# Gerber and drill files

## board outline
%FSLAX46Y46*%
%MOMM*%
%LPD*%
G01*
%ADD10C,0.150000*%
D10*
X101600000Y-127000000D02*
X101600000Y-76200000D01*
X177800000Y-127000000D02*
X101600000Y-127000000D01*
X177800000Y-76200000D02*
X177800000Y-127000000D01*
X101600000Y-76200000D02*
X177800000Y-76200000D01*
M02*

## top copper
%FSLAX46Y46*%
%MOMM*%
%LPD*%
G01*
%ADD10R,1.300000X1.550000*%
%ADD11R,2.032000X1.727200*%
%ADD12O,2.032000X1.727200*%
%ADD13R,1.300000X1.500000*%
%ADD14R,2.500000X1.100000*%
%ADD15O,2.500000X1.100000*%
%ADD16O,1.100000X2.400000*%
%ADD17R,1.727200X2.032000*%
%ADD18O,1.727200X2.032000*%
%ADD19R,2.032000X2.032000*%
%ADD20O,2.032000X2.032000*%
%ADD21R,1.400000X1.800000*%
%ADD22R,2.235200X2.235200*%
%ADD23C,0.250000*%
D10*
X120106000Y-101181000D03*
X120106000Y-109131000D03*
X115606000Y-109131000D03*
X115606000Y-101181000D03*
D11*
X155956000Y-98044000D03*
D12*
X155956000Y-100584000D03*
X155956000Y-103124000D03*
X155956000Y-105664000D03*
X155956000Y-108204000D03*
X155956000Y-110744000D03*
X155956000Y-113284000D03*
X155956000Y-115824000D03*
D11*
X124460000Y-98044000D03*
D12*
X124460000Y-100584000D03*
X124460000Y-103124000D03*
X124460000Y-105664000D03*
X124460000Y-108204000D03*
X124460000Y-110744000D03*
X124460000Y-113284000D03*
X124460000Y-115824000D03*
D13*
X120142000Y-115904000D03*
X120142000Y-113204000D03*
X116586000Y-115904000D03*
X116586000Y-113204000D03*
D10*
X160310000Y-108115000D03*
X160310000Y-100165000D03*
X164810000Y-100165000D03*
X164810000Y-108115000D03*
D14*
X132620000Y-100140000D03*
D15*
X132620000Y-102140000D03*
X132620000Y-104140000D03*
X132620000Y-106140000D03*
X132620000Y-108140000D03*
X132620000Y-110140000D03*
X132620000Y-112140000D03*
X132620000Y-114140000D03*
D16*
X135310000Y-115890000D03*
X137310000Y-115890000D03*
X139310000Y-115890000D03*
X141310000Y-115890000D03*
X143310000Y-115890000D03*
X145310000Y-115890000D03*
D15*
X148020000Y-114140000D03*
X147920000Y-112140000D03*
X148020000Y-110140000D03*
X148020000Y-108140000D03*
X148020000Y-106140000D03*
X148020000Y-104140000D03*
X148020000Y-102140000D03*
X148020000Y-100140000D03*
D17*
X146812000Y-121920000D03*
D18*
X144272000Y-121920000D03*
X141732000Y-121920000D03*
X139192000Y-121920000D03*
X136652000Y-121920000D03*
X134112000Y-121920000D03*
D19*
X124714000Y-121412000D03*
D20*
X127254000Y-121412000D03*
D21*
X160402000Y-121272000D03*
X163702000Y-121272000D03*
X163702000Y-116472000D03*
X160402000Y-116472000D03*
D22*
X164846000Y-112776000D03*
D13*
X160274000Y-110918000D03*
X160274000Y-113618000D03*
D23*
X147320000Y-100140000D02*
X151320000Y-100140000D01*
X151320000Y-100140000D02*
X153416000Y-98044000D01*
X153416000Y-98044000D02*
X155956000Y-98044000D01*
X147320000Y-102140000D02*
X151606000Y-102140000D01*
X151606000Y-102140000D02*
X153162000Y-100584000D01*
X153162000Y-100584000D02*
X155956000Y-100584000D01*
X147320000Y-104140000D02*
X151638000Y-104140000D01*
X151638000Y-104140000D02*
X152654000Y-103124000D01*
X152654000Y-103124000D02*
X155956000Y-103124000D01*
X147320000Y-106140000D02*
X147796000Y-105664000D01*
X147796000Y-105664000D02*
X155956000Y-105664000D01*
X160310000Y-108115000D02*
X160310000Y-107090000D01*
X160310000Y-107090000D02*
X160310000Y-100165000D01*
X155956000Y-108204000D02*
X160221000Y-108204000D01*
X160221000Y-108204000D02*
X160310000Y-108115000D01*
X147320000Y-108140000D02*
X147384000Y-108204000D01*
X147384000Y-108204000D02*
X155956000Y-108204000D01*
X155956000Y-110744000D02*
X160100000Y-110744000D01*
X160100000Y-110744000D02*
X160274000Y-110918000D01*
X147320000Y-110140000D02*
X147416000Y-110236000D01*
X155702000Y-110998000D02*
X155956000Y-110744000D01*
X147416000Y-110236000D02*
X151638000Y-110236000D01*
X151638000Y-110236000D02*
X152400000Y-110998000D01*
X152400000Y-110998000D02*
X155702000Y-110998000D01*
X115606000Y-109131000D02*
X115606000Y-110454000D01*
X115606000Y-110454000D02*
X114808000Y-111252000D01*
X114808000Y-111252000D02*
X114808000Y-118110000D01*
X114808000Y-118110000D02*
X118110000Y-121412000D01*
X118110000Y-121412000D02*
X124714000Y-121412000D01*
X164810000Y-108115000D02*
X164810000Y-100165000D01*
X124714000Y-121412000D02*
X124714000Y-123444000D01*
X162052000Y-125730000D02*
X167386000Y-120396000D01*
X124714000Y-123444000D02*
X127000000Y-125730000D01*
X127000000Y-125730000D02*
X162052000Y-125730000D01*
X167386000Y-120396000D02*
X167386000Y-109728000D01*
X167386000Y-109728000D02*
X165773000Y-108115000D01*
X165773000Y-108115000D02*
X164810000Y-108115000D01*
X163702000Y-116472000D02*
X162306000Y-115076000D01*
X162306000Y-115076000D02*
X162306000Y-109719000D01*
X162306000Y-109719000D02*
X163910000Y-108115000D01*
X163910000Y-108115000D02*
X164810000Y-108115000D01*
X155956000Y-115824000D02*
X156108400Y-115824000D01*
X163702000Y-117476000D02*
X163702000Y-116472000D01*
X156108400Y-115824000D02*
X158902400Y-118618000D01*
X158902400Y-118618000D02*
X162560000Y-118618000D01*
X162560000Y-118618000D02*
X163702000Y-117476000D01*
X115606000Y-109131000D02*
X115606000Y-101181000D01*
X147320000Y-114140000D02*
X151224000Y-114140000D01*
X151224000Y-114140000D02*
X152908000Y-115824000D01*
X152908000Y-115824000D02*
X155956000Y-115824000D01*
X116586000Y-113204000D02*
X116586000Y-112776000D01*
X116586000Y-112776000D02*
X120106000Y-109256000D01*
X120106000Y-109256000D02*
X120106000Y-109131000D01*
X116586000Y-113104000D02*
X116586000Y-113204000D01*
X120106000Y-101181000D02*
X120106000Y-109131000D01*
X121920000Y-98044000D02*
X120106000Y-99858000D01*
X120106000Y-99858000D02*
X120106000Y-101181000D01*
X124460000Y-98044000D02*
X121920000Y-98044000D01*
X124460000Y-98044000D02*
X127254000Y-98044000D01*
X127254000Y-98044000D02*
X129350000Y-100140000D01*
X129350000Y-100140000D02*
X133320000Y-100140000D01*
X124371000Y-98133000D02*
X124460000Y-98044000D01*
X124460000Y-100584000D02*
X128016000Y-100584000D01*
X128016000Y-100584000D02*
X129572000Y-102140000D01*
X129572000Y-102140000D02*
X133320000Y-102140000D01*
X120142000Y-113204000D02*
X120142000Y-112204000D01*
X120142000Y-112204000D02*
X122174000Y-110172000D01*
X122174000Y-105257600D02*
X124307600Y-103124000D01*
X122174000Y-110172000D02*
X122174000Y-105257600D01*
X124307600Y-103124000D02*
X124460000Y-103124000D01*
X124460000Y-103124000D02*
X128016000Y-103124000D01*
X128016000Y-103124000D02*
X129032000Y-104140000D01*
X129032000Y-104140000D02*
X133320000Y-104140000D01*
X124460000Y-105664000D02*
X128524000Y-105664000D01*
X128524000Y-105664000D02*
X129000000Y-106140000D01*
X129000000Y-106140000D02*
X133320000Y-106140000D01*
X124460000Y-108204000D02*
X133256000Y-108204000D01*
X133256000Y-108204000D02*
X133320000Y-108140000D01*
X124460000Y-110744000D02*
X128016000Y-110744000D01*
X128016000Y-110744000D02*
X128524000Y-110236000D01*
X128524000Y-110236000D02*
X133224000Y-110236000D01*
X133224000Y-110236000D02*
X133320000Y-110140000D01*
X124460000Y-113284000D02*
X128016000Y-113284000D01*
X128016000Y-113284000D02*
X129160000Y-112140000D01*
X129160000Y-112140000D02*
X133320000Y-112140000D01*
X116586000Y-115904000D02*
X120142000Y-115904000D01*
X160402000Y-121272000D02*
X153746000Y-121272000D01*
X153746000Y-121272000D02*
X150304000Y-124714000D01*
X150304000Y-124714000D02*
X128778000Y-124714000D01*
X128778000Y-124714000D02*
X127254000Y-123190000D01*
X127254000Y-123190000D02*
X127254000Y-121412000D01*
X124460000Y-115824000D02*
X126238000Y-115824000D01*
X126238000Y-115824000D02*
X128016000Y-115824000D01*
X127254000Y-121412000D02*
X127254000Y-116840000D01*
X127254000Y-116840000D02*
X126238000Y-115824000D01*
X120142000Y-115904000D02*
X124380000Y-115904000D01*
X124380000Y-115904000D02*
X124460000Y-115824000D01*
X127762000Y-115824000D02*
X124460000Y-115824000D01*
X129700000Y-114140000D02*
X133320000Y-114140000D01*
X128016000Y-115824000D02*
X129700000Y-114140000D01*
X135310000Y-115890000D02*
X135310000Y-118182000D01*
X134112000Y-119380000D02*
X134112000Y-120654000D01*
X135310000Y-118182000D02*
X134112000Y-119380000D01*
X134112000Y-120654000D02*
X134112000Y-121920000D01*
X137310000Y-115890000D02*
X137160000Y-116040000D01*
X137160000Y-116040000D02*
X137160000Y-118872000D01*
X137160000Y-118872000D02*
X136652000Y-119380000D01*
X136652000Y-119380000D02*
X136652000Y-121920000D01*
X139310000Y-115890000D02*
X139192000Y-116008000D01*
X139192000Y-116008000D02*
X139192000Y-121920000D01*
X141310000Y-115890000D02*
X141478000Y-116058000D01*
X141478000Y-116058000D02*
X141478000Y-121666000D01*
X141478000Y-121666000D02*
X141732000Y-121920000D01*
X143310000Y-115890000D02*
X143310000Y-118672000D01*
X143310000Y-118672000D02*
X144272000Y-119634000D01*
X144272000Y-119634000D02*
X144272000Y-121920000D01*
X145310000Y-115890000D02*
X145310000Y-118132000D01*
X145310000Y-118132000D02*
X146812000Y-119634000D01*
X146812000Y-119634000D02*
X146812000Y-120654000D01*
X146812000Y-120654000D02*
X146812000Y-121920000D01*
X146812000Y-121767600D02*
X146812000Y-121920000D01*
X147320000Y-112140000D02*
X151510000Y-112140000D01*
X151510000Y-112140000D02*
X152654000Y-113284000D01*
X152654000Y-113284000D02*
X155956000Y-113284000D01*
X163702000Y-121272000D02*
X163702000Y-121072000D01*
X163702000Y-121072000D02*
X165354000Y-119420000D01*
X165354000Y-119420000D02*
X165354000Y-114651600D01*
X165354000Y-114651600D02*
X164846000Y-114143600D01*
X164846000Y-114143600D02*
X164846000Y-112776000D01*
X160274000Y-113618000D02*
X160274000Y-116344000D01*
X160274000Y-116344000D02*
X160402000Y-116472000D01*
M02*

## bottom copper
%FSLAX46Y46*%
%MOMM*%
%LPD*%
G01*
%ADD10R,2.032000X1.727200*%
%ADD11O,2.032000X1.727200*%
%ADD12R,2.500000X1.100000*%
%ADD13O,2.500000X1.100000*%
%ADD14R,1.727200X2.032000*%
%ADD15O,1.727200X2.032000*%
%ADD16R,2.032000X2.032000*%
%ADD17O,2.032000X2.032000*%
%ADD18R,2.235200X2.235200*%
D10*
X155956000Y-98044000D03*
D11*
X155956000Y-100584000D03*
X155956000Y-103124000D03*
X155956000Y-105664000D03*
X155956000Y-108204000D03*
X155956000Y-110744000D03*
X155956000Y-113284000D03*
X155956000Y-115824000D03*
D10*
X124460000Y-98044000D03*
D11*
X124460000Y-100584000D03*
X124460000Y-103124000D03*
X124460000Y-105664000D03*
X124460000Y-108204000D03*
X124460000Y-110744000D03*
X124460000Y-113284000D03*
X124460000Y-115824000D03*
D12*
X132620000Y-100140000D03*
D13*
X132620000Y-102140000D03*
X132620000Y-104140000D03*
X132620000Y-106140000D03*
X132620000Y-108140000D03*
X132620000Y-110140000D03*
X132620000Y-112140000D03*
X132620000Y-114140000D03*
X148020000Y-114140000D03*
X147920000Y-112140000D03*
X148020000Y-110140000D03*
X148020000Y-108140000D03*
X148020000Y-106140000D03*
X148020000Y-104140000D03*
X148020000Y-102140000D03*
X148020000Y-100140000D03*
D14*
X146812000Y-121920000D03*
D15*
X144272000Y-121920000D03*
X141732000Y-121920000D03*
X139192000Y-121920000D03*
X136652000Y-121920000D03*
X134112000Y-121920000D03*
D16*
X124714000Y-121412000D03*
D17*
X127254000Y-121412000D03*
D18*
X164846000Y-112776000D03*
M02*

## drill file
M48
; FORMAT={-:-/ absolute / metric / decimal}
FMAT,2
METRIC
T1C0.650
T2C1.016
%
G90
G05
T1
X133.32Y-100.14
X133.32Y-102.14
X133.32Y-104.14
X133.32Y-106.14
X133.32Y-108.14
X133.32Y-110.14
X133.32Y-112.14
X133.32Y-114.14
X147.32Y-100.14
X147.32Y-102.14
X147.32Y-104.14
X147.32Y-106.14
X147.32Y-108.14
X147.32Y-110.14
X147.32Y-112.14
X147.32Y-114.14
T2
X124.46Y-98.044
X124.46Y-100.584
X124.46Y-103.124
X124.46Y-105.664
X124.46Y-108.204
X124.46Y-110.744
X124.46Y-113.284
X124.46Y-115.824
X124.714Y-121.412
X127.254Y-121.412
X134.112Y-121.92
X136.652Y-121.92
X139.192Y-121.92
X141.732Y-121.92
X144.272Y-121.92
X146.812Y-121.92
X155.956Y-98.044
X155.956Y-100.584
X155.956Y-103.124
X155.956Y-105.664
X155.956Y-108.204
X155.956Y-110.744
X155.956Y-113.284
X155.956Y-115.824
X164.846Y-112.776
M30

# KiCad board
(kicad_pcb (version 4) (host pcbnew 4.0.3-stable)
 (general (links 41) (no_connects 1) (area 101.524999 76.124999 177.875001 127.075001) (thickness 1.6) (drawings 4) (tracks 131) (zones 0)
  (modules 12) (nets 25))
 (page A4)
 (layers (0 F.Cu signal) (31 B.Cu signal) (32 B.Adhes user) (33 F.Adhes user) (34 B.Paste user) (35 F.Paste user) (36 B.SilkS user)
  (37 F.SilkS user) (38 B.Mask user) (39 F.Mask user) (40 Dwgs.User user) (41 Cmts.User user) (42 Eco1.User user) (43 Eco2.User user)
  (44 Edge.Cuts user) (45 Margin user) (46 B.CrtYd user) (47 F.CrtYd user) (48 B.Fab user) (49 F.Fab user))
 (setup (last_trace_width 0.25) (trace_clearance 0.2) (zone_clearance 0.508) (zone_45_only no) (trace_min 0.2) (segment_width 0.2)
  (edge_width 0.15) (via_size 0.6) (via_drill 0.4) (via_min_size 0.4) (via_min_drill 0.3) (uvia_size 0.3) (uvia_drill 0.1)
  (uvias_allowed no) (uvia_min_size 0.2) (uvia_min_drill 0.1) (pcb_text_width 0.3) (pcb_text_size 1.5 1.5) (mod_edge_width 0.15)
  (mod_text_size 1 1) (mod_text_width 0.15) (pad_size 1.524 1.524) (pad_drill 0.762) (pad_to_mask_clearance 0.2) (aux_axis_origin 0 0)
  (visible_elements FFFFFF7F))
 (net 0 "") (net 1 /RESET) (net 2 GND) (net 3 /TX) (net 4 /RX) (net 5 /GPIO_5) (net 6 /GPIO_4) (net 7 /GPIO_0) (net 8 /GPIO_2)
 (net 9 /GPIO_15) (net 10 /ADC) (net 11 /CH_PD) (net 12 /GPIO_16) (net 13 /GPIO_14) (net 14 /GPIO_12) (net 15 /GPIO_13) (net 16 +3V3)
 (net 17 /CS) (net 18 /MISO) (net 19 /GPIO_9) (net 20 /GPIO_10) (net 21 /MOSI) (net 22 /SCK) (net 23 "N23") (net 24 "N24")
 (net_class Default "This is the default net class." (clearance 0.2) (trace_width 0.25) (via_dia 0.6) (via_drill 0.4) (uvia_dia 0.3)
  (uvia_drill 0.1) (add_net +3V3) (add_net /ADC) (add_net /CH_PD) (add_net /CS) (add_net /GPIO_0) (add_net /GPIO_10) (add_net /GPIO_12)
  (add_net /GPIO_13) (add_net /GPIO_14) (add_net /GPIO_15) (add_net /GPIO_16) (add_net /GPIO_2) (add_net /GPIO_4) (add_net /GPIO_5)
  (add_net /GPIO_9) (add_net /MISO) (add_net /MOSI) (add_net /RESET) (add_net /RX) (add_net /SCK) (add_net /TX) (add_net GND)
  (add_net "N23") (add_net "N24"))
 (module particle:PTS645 (layer F.Cu) (at 117.856 105.156 270)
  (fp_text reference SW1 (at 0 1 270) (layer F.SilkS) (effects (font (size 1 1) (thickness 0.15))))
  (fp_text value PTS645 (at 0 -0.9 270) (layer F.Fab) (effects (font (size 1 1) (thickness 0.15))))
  (pad 1 smd rect (at -3.975 -2.25 270) (size 1.55 1.3) (layers F.Cu F.Paste F.Mask) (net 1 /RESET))
  (pad 1 smd rect (at 3.975 -2.25 270) (size 1.55 1.3) (layers F.Cu F.Paste F.Mask) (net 1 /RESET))
  (pad 4 smd rect (at 3.975 2.25 270) (size 1.55 1.3) (layers F.Cu F.Paste F.Mask) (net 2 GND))
  (pad 4 smd rect (at -3.975 2.25 270) (size 1.55 1.3) (layers F.Cu F.Paste F.Mask) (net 2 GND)))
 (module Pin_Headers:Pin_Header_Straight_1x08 (layer F.Cu) (at 155.956 98.044)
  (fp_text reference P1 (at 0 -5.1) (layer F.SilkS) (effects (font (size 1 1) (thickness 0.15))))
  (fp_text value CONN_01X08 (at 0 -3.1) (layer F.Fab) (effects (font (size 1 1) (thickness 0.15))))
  (pad 1 thru_hole rect (at 0 0) (size 2.032 1.7272) (drill 1.016) (layers *.Cu *.Mask F.SilkS) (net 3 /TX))
  (pad 2 thru_hole oval (at 0 2.54) (size 2.032 1.7272) (drill 1.016) (layers *.Cu *.Mask F.SilkS) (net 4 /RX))
  (pad 3 thru_hole oval (at 0 5.08) (size 2.032 1.7272) (drill 1.016) (layers *.Cu *.Mask F.SilkS) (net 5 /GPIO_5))
  (pad 4 thru_hole oval (at 0 7.62) (size 2.032 1.7272) (drill 1.016) (layers *.Cu *.Mask F.SilkS) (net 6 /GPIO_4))
  (pad 5 thru_hole oval (at 0 10.16) (size 2.032 1.7272) (drill 1.016) (layers *.Cu *.Mask F.SilkS) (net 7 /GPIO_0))
  (pad 6 thru_hole oval (at 0 12.7) (size 2.032 1.7272) (drill 1.016) (layers *.Cu *.Mask F.SilkS) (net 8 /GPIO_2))
  (pad 7 thru_hole oval (at 0 15.24) (size 2.032 1.7272) (drill 1.016) (layers *.Cu *.Mask F.SilkS) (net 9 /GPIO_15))
  (pad 8 thru_hole oval (at 0 17.78) (size 2.032 1.7272) (drill 1.016) (layers *.Cu *.Mask F.SilkS) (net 2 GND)))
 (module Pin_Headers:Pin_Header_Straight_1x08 (layer F.Cu) (at 124.46 98.044)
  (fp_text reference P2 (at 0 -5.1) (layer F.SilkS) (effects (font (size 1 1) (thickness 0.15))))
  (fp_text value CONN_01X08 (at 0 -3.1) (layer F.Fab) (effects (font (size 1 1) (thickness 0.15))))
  (pad 1 thru_hole rect (at 0 0) (size 2.032 1.7272) (drill 1.016) (layers *.Cu *.Mask F.SilkS) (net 1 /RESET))
  (pad 2 thru_hole oval (at 0 2.54) (size 2.032 1.7272) (drill 1.016) (layers *.Cu *.Mask F.SilkS) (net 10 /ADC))
  (pad 3 thru_hole oval (at 0 5.08) (size 2.032 1.7272) (drill 1.016) (layers *.Cu *.Mask F.SilkS) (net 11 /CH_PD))
  (pad 4 thru_hole oval (at 0 7.62) (size 2.032 1.7272) (drill 1.016) (layers *.Cu *.Mask F.SilkS) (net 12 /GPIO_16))
  (pad 5 thru_hole oval (at 0 10.16) (size 2.032 1.7272) (drill 1.016) (layers *.Cu *.Mask F.SilkS) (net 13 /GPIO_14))
  (pad 6 thru_hole oval (at 0 12.7) (size 2.032 1.7272) (drill 1.016) (layers *.Cu *.Mask F.SilkS) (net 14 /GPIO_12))
  (pad 7 thru_hole oval (at 0 15.24) (size 2.032 1.7272) (drill 1.016) (layers *.Cu *.Mask F.SilkS) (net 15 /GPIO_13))
  (pad 8 thru_hole oval (at 0 17.78) (size 2.032 1.7272) (drill 1.016) (layers *.Cu *.Mask F.SilkS) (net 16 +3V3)))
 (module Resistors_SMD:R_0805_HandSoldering (layer F.Cu) (at 120.142 114.554 90)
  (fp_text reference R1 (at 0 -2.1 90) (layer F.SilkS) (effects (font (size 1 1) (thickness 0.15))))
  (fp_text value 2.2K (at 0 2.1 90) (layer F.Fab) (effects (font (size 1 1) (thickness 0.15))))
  (pad 1 smd rect (at -1.35 0 90) (size 1.5 1.3) (layers F.Cu F.Paste F.Mask) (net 16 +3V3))
  (pad 2 smd rect (at 1.35 0 90) (size 1.5 1.3) (layers F.Cu F.Paste F.Mask) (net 11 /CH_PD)))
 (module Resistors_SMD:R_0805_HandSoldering (layer F.Cu) (at 116.586 114.554 90)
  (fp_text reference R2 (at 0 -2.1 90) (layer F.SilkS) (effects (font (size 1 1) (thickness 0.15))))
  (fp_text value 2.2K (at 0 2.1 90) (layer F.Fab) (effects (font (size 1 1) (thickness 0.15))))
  (pad 1 smd rect (at -1.35 0 90) (size 1.5 1.3) (layers F.Cu F.Paste F.Mask) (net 16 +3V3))
  (pad 2 smd rect (at 1.35 0 90) (size 1.5 1.3) (layers F.Cu F.Paste F.Mask) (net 1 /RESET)))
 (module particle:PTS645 (layer F.Cu) (at 162.56 104.14 90)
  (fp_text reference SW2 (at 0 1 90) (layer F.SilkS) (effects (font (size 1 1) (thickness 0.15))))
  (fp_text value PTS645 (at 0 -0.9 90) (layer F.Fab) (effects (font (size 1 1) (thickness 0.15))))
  (pad 1 smd rect (at -3.975 -2.25 90) (size 1.55 1.3) (layers F.Cu F.Paste F.Mask) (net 7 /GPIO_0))
  (pad 1 smd rect (at 3.975 -2.25 90) (size 1.55 1.3) (layers F.Cu F.Paste F.Mask) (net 7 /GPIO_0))
  (pad 4 smd rect (at 3.975 2.25 90) (size 1.55 1.3) (layers F.Cu F.Paste F.Mask) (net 2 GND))
  (pad 4 smd rect (at -3.975 2.25 90) (size 1.55 1.3) (layers F.Cu F.Paste F.Mask) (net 2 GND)))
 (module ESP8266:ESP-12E (layer F.Cu) (at 133.32 100.14)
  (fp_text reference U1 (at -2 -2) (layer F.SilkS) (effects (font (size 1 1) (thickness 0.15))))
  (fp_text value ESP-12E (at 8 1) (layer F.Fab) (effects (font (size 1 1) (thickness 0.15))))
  (pad 1 thru_hole rect (at 0 0) (size 2.5 1.1) (drill 0.65 (offset -0.7 0)) (layers *.Cu *.Mask F.SilkS) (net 1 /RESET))
  (pad 2 thru_hole oval (at 0 2) (size 2.5 1.1) (drill 0.65 (offset -0.7 0)) (layers *.Cu *.Mask F.SilkS) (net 10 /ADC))
  (pad 3 thru_hole oval (at 0 4) (size 2.5 1.1) (drill 0.65 (offset -0.7 0)) (layers *.Cu *.Mask F.SilkS) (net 11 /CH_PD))
  (pad 4 thru_hole oval (at 0 6) (size 2.5 1.1) (drill 0.65 (offset -0.7 0)) (layers *.Cu *.Mask F.SilkS) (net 12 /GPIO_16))
  (pad 5 thru_hole oval (at 0 8) (size 2.5 1.1) (drill 0.65 (offset -0.7 0)) (layers *.Cu *.Mask F.SilkS) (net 13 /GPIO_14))
  (pad 6 thru_hole oval (at 0 10) (size 2.5 1.1) (drill 0.65 (offset -0.7 0)) (layers *.Cu *.Mask F.SilkS) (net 14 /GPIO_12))
  (pad 7 thru_hole oval (at 0 12) (size 2.5 1.1) (drill 0.65 (offset -0.7 0)) (layers *.Cu *.Mask F.SilkS) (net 15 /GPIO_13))
  (pad 8 thru_hole oval (at 0 14) (size 2.5 1.1) (drill 0.65 (offset -0.7 0)) (layers *.Cu *.Mask F.SilkS) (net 16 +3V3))
  (pad 9 smd oval (at 1.99 15.75 90) (size 2.4 1.1) (layers F.Cu F.Paste F.Mask) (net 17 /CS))
  (pad 10 smd oval (at 3.99 15.75 90) (size 2.4 1.1) (layers F.Cu F.Paste F.Mask) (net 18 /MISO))
  (pad 11 smd oval (at 5.99 15.75 90) (size 2.4 1.1) (layers F.Cu F.Paste F.Mask) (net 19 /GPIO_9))
  (pad 12 smd oval (at 7.99 15.75 90) (size 2.4 1.1) (layers F.Cu F.Paste F.Mask) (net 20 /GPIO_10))
  (pad 13 smd oval (at 9.99 15.75 90) (size 2.4 1.1) (layers F.Cu F.Paste F.Mask) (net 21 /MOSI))
  (pad 14 smd oval (at 11.99 15.75 90) (size 2.4 1.1) (layers F.Cu F.Paste F.Mask) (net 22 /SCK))
  (pad 15 thru_hole oval (at 14 14) (size 2.5 1.1) (drill 0.65 (offset 0.7 0)) (layers *.Cu *.Mask F.SilkS) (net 2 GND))
  (pad 16 thru_hole oval (at 14 12) (size 2.5 1.1) (drill 0.65 (offset 0.6 0)) (layers *.Cu *.Mask F.SilkS) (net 9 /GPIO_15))
  (pad 17 thru_hole oval (at 14 10) (size 2.5 1.1) (drill 0.65 (offset 0.7 0)) (layers *.Cu *.Mask F.SilkS) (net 8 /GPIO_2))
  (pad 18 thru_hole oval (at 14 8) (size 2.5 1.1) (drill 0.65 (offset 0.7 0)) (layers *.Cu *.Mask F.SilkS) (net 7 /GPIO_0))
  (pad 19 thru_hole oval (at 14 6) (size 2.5 1.1) (drill 0.65 (offset 0.7 0)) (layers *.Cu *.Mask F.SilkS) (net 6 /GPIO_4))
  (pad 20 thru_hole oval (at 14 4) (size 2.5 1.1) (drill 0.65 (offset 0.7 0)) (layers *.Cu *.Mask F.SilkS) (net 5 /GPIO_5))
  (pad 21 thru_hole oval (at 14 2) (size 2.5 1.1) (drill 0.65 (offset 0.7 0)) (layers *.Cu *.Mask F.SilkS) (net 4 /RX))
  (pad 22 thru_hole oval (at 14 0) (size 2.5 1.1) (drill 0.65 (offset 0.7 0)) (layers *.Cu *.Mask F.SilkS) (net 3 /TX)))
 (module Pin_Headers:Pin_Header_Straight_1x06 (layer F.Cu) (at 146.812 121.92 270)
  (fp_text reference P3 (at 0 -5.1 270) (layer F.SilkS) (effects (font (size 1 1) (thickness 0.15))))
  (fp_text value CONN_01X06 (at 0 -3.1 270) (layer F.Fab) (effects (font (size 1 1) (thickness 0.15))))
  (pad 1 thru_hole rect (at 0 0 270) (size 2.032 1.7272) (drill 1.016) (layers *.Cu *.Mask F.SilkS) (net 22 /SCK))
  (pad 2 thru_hole oval (at 0 2.54 270) (size 2.032 1.7272) (drill 1.016) (layers *.Cu *.Mask F.SilkS) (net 21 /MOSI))
  (pad 3 thru_hole oval (at 0 5.08 270) (size 2.032 1.7272) (drill 1.016) (layers *.Cu *.Mask F.SilkS) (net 20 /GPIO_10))
  (pad 4 thru_hole oval (at 0 7.62 270) (size 2.032 1.7272) (drill 1.016) (layers *.Cu *.Mask F.SilkS) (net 19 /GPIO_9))
  (pad 5 thru_hole oval (at 0 10.16 270) (size 2.032 1.7272) (drill 1.016) (layers *.Cu *.Mask F.SilkS) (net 18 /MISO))
  (pad 6 thru_hole oval (at 0 12.7 270) (size 2.032 1.7272) (drill 1.016) (layers *.Cu *.Mask F.SilkS) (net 17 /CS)))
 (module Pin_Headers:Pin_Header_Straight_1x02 (layer F.Cu) (at 124.714 121.412 90)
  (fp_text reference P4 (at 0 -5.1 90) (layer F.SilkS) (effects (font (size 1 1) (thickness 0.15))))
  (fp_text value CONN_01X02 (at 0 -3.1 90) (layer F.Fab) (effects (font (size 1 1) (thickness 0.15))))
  (pad 1 thru_hole rect (at 0 0 90) (size 2.032 2.032) (drill 1.016) (layers *.Cu *.Mask F.SilkS) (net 2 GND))
  (pad 2 thru_hole oval (at 0 2.54 90) (size 2.032 2.032) (drill 1.016) (layers *.Cu *.Mask F.SilkS) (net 16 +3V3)))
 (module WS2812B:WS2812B (layer F.Cu) (at 162.052 118.872 180)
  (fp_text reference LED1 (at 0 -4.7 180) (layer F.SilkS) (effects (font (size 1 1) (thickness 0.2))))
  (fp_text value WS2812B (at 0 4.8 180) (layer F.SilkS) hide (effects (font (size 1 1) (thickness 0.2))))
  (pad 1 smd rect (at 1.65 -2.4 180) (size 1.4 1.8) (layers F.Cu F.Paste F.Mask) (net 16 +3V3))
  (pad 2 smd rect (at -1.65 -2.4 180) (size 1.4 1.8) (layers F.Cu F.Paste F.Mask) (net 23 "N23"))
  (pad 3 smd rect (at -1.65 2.4 180) (size 1.4 1.8) (layers F.Cu F.Paste F.Mask) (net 2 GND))
  (pad 4 smd rect (at 1.65 2.4 180) (size 1.4 1.8) (layers F.Cu F.Paste F.Mask) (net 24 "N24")))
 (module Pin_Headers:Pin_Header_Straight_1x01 (layer F.Cu) (at 164.846 112.776)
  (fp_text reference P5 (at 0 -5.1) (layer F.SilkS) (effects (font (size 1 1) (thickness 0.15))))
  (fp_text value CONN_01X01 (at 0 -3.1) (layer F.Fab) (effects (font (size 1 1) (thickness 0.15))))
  (pad 1 thru_hole rect (at 0 0) (size 2.2352 2.2352) (drill 1.016) (layers *.Cu *.Mask F.SilkS) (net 23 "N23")))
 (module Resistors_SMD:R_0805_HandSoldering (layer F.Cu) (at 160.274 112.268 270)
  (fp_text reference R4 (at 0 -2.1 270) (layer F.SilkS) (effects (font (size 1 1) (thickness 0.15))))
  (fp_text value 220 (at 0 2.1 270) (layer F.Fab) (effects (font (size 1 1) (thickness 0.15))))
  (pad 1 smd rect (at -1.35 0 270) (size 1.5 1.3) (layers F.Cu F.Paste F.Mask) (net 8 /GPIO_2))
  (pad 2 smd rect (at 1.35 0 270) (size 1.5 1.3) (layers F.Cu F.Paste F.Mask) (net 24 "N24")))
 (gr_line (start 101.6 127) (end 101.6 76.2) (layer Edge.Cuts) (width 0.15))
 (gr_line (start 177.8 127) (end 101.6 127) (layer Edge.Cuts) (width 0.15))
 (gr_line (start 177.8 76.2) (end 177.8 127) (layer Edge.Cuts) (width 0.15))
 (gr_line (start 101.6 76.2) (end 177.8 76.2) (layer Edge.Cuts) (width 0.15))
 (segment (start 147.32 100.14) (end 151.32 100.14) (width 0.25) (layer F.Cu) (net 3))
 (segment (start 151.32 100.14) (end 153.416 98.044) (width 0.25) (layer F.Cu) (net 3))
 (segment (start 153.416 98.044) (end 155.956 98.044) (width 0.25) (layer F.Cu) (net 3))
 (segment (start 147.32 102.14) (end 151.606 102.14) (width 0.25) (layer F.Cu) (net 4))
 (segment (start 151.606 102.14) (end 153.162 100.584) (width 0.25) (layer F.Cu) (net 4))
 (segment (start 153.162 100.584) (end 155.956 100.584) (width 0.25) (layer F.Cu) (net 4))
 (segment (start 147.32 104.14) (end 151.638 104.14) (width 0.25) (layer F.Cu) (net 5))
 (segment (start 151.638 104.14) (end 152.654 103.124) (width 0.25) (layer F.Cu) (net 5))
 (segment (start 152.654 103.124) (end 155.956 103.124) (width 0.25) (layer F.Cu) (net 5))
 (segment (start 147.32 106.14) (end 147.796 105.664) (width 0.25) (layer F.Cu) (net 6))
 (segment (start 147.796 105.664) (end 155.956 105.664) (width 0.25) (layer F.Cu) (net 6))
 (segment (start 160.31 108.115) (end 160.31 107.09) (width 0.25) (layer F.Cu) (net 7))
 (segment (start 160.31 107.09) (end 160.31 100.165) (width 0.25) (layer F.Cu) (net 7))
 (segment (start 155.956 108.204) (end 160.221 108.204) (width 0.25) (layer F.Cu) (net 7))
 (segment (start 160.221 108.204) (end 160.31 108.115) (width 0.25) (layer F.Cu) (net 7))
 (segment (start 147.32 108.14) (end 147.384 108.204) (width 0.25) (layer F.Cu) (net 7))
 (segment (start 147.384 108.204) (end 155.956 108.204) (width 0.25) (layer F.Cu) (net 7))
 (segment (start 155.956 110.744) (end 160.1 110.744) (width 0.25) (layer F.Cu) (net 8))
 (segment (start 160.1 110.744) (end 160.274 110.918) (width 0.25) (layer F.Cu) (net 8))
 (segment (start 147.32 110.14) (end 147.416 110.236) (width 0.25) (layer F.Cu) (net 8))
 (segment (start 155.702 110.998) (end 155.956 110.744) (width 0.25) (layer F.Cu) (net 8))
 (segment (start 147.416 110.236) (end 151.638 110.236) (width 0.25) (layer F.Cu) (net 8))
 (segment (start 151.638 110.236) (end 152.4 110.998) (width 0.25) (layer F.Cu) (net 8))
 (segment (start 152.4 110.998) (end 155.702 110.998) (width 0.25) (layer F.Cu) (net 8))
 (segment (start 115.606 109.131) (end 115.606 110.454) (width 0.25) (layer F.Cu) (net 2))
 (segment (start 115.606 110.454) (end 114.808 111.252) (width 0.25) (layer F.Cu) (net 2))
 (segment (start 114.808 111.252) (end 114.808 118.11) (width 0.25) (layer F.Cu) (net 2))
 (segment (start 114.808 118.11) (end 118.11 121.412) (width 0.25) (layer F.Cu) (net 2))
 (segment (start 118.11 121.412) (end 124.714 121.412) (width 0.25) (layer F.Cu) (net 2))
 (segment (start 164.81 108.115) (end 164.81 100.165) (width 0.25) (layer F.Cu) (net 2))
 (segment (start 124.714 121.412) (end 124.714 123.444) (width 0.25) (layer F.Cu) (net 2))
 (segment (start 162.052 125.73) (end 167.386 120.396) (width 0.25) (layer F.Cu) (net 2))
 (segment (start 124.714 123.444) (end 127 125.73) (width 0.25) (layer F.Cu) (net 2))
 (segment (start 127 125.73) (end 162.052 125.73) (width 0.25) (layer F.Cu) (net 2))
 (segment (start 167.386 120.396) (end 167.386 109.728) (width 0.25) (layer F.Cu) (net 2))
 (segment (start 167.386 109.728) (end 165.773 108.115) (width 0.25) (layer F.Cu) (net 2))
 (segment (start 165.773 108.115) (end 164.81 108.115) (width 0.25) (layer F.Cu) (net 2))
 (segment (start 163.702 116.472) (end 162.306 115.076) (width 0.25) (layer F.Cu) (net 2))
 (segment (start 162.306 115.076) (end 162.306 109.719) (width 0.25) (layer F.Cu) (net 2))
 (segment (start 162.306 109.719) (end 163.91 108.115) (width 0.25) (layer F.Cu) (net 2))
 (segment (start 163.91 108.115) (end 164.81 108.115) (width 0.25) (layer F.Cu) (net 2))
 (segment (start 155.956 115.824) (end 156.1084 115.824) (width 0.25) (layer F.Cu) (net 2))
 (segment (start 163.702 117.476) (end 163.702 116.472) (width 0.25) (layer F.Cu) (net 2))
 (segment (start 156.1084 115.824) (end 158.9024 118.618) (width 0.25) (layer F.Cu) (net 2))
 (segment (start 158.9024 118.618) (end 162.56 118.618) (width 0.25) (layer F.Cu) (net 2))
 (segment (start 162.56 118.618) (end 163.702 117.476) (width 0.25) (layer F.Cu) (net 2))
 (segment (start 115.606 109.131) (end 115.606 101.181) (width 0.25) (layer F.Cu) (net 2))
 (segment (start 147.32 114.14) (end 151.224 114.14) (width 0.25) (layer F.Cu) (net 2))
 (segment (start 151.224 114.14) (end 152.908 115.824) (width 0.25) (layer F.Cu) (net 2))
 (segment (start 152.908 115.824) (end 155.956 115.824) (width 0.25) (layer F.Cu) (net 2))
 (segment (start 116.586 113.204) (end 116.586 112.776) (width 0.25) (layer F.Cu) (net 1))
 (segment (start 116.586 112.776) (end 120.106 109.256) (width 0.25) (layer F.Cu) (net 1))
 (segment (start 120.106 109.256) (end 120.106 109.131) (width 0.25) (layer F.Cu) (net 1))
 (segment (start 116.586 113.104) (end 116.586 113.204) (width 0.25) (layer F.Cu) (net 1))
 (segment (start 120.106 101.181) (end 120.106 109.131) (width 0.25) (layer F.Cu) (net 1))
 (segment (start 121.92 98.044) (end 120.106 99.858) (width 0.25) (layer F.Cu) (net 1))
 (segment (start 120.106 99.858) (end 120.106 101.181) (width 0.25) (layer F.Cu) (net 1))
 (segment (start 124.46 98.044) (end 121.92 98.044) (width 0.25) (layer F.Cu) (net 1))
 (segment (start 124.46 98.044) (end 127.254 98.044) (width 0.25) (layer F.Cu) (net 1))
 (segment (start 127.254 98.044) (end 129.35 100.14) (width 0.25) (layer F.Cu) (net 1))
 (segment (start 129.35 100.14) (end 133.32 100.14) (width 0.25) (layer F.Cu) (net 1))
 (segment (start 124.371 98.133) (end 124.46 98.044) (width 0.25) (layer F.Cu) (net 1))
 (segment (start 124.46 100.584) (end 128.016 100.584) (width 0.25) (layer F.Cu) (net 10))
 (segment (start 128.016 100.584) (end 129.572 102.14) (width 0.25) (layer F.Cu) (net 10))
 (segment (start 129.572 102.14) (end 133.32 102.14) (width 0.25) (layer F.Cu) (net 10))
 (segment (start 120.142 113.204) (end 120.142 112.204) (width 0.25) (layer F.Cu) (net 11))
 (segment (start 120.142 112.204) (end 122.174 110.172) (width 0.25) (layer F.Cu) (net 11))
 (segment (start 122.174 105.2576) (end 124.3076 103.124) (width 0.25) (layer F.Cu) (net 11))
 (segment (start 122.174 110.172) (end 122.174 105.2576) (width 0.25) (layer F.Cu) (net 11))
 (segment (start 124.3076 103.124) (end 124.46 103.124) (width 0.25) (layer F.Cu) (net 11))
 (segment (start 124.46 103.124) (end 128.016 103.124) (width 0.25) (layer F.Cu) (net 11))
 (segment (start 128.016 103.124) (end 129.032 104.14) (width 0.25) (layer F.Cu) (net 11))
 (segment (start 129.032 104.14) (end 133.32 104.14) (width 0.25) (layer F.Cu) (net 11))
 (segment (start 124.46 105.664) (end 128.524 105.664) (width 0.25) (layer F.Cu) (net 12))
 (segment (start 128.524 105.664) (end 129 106.14) (width 0.25) (layer F.Cu) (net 12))
 (segment (start 129 106.14) (end 133.32 106.14) (width 0.25) (layer F.Cu) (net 12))
 (segment (start 124.46 108.204) (end 133.256 108.204) (width 0.25) (layer F.Cu) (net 13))
 (segment (start 133.256 108.204) (end 133.32 108.14) (width 0.25) (layer F.Cu) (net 13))
 (segment (start 124.46 110.744) (end 128.016 110.744) (width 0.25) (layer F.Cu) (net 14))
 (segment (start 128.016 110.744) (end 128.524 110.236) (width 0.25) (layer F.Cu) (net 14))
 (segment (start 128.524 110.236) (end 133.224 110.236) (width 0.25) (layer F.Cu) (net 14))
 (segment (start 133.224 110.236) (end 133.32 110.14) (width 0.25) (layer F.Cu) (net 14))
 (segment (start 124.46 113.284) (end 128.016 113.284) (width 0.25) (layer F.Cu) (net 15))
 (segment (start 128.016 113.284) (end 129.16 112.14) (width 0.25) (layer F.Cu) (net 15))
 (segment (start 129.16 112.14) (end 133.32 112.14) (width 0.25) (layer F.Cu) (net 15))
 (segment (start 116.586 115.904) (end 120.142 115.904) (width 0.25) (layer F.Cu) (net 16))
 (segment (start 160.402 121.272) (end 153.746 121.272) (width 0.25) (layer F.Cu) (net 16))
 (segment (start 153.746 121.272) (end 150.304 124.714) (width 0.25) (layer F.Cu) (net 16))
 (segment (start 150.304 124.714) (end 128.778 124.714) (width 0.25) (layer F.Cu) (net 16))
 (segment (start 128.778 124.714) (end 127.254 123.19) (width 0.25) (layer F.Cu) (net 16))
 (segment (start 127.254 123.19) (end 127.254 121.412) (width 0.25) (layer F.Cu) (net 16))
 (segment (start 124.46 115.824) (end 126.238 115.824) (width 0.25) (layer F.Cu) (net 16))
 (segment (start 126.238 115.824) (end 128.016 115.824) (width 0.25) (layer F.Cu) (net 16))
 (segment (start 127.254 121.412) (end 127.254 116.84) (width 0.25) (layer F.Cu) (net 16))
 (segment (start 127.254 116.84) (end 126.238 115.824) (width 0.25) (layer F.Cu) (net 16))
 (segment (start 120.142 115.904) (end 124.38 115.904) (width 0.25) (layer F.Cu) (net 16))
 (segment (start 124.38 115.904) (end 124.46 115.824) (width 0.25) (layer F.Cu) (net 16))
 (segment (start 127.762 115.824) (end 124.46 115.824) (width 0.25) (layer F.Cu) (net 16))
 (segment (start 129.7 114.14) (end 133.32 114.14) (width 0.25) (layer F.Cu) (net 16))
 (segment (start 128.016 115.824) (end 129.7 114.14) (width 0.25) (layer F.Cu) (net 16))
 (segment (start 135.31 115.89) (end 135.31 118.182) (width 0.25) (layer F.Cu) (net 17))
 (segment (start 134.112 119.38) (end 134.112 120.654) (width 0.25) (layer F.Cu) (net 17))
 (segment (start 135.31 118.182) (end 134.112 119.38) (width 0.25) (layer F.Cu) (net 17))
 (segment (start 134.112 120.654) (end 134.112 121.92) (width 0.25) (layer F.Cu) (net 17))
 (segment (start 137.31 115.89) (end 137.16 116.04) (width 0.25) (layer F.Cu) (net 18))
 (segment (start 137.16 116.04) (end 137.16 118.872) (width 0.25) (layer F.Cu) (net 18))
 (segment (start 137.16 118.872) (end 136.652 119.38) (width 0.25) (layer F.Cu) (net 18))
 (segment (start 136.652 119.38) (end 136.652 121.92) (width 0.25) (layer F.Cu) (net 18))
 (segment (start 139.31 115.89) (end 139.192 116.008) (width 0.25) (layer F.Cu) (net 19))
 (segment (start 139.192 116.008) (end 139.192 121.92) (width 0.25) (layer F.Cu) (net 19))
 (segment (start 141.31 115.89) (end 141.478 116.058) (width 0.25) (layer F.Cu) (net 20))
 (segment (start 141.478 116.058) (end 141.478 121.666) (width 0.25) (layer F.Cu) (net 20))
 (segment (start 141.478 121.666) (end 141.732 121.92) (width 0.25) (layer F.Cu) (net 20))
 (segment (start 143.31 115.89) (end 143.31 118.672) (width 0.25) (layer F.Cu) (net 21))
 (segment (start 143.31 118.672) (end 144.272 119.634) (width 0.25) (layer F.Cu) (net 21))
 (segment (start 144.272 119.634) (end 144.272 121.92) (width 0.25) (layer F.Cu) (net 21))
 (segment (start 145.31 115.89) (end 145.31 118.132) (width 0.25) (layer F.Cu) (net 22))
 (segment (start 145.31 118.132) (end 146.812 119.634) (width 0.25) (layer F.Cu) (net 22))
 (segment (start 146.812 119.634) (end 146.812 120.654) (width 0.25) (layer F.Cu) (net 22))
 (segment (start 146.812 120.654) (end 146.812 121.92) (width 0.25) (layer F.Cu) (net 22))
 (segment (start 146.812 121.7676) (end 146.812 121.92) (width 0.25) (layer F.Cu) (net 22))
 (segment (start 147.32 112.14) (end 151.51 112.14) (width 0.25) (layer F.Cu) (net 9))
 (segment (start 151.51 112.14) (end 152.654 113.284) (width 0.25) (layer F.Cu) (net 9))
 (segment (start 152.654 113.284) (end 155.956 113.284) (width 0.25) (layer F.Cu) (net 9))
 (segment (start 163.702 121.272) (end 163.702 121.072) (width 0.25) (layer F.Cu) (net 23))
 (segment (start 163.702 121.072) (end 165.354 119.42) (width 0.25) (layer F.Cu) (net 23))
 (segment (start 165.354 119.42) (end 165.354 114.6516) (width 0.25) (layer F.Cu) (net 23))
 (segment (start 165.354 114.6516) (end 164.846 114.1436) (width 0.25) (layer F.Cu) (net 23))
 (segment (start 164.846 114.1436) (end 164.846 112.776) (width 0.25) (layer F.Cu) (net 23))
 (segment (start 160.274 113.618) (end 160.274 116.344) (width 0.25) (layer F.Cu) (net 24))
 (segment (start 160.274 116.344) (end 160.402 116.472) (width 0.25) (layer F.Cu) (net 24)))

